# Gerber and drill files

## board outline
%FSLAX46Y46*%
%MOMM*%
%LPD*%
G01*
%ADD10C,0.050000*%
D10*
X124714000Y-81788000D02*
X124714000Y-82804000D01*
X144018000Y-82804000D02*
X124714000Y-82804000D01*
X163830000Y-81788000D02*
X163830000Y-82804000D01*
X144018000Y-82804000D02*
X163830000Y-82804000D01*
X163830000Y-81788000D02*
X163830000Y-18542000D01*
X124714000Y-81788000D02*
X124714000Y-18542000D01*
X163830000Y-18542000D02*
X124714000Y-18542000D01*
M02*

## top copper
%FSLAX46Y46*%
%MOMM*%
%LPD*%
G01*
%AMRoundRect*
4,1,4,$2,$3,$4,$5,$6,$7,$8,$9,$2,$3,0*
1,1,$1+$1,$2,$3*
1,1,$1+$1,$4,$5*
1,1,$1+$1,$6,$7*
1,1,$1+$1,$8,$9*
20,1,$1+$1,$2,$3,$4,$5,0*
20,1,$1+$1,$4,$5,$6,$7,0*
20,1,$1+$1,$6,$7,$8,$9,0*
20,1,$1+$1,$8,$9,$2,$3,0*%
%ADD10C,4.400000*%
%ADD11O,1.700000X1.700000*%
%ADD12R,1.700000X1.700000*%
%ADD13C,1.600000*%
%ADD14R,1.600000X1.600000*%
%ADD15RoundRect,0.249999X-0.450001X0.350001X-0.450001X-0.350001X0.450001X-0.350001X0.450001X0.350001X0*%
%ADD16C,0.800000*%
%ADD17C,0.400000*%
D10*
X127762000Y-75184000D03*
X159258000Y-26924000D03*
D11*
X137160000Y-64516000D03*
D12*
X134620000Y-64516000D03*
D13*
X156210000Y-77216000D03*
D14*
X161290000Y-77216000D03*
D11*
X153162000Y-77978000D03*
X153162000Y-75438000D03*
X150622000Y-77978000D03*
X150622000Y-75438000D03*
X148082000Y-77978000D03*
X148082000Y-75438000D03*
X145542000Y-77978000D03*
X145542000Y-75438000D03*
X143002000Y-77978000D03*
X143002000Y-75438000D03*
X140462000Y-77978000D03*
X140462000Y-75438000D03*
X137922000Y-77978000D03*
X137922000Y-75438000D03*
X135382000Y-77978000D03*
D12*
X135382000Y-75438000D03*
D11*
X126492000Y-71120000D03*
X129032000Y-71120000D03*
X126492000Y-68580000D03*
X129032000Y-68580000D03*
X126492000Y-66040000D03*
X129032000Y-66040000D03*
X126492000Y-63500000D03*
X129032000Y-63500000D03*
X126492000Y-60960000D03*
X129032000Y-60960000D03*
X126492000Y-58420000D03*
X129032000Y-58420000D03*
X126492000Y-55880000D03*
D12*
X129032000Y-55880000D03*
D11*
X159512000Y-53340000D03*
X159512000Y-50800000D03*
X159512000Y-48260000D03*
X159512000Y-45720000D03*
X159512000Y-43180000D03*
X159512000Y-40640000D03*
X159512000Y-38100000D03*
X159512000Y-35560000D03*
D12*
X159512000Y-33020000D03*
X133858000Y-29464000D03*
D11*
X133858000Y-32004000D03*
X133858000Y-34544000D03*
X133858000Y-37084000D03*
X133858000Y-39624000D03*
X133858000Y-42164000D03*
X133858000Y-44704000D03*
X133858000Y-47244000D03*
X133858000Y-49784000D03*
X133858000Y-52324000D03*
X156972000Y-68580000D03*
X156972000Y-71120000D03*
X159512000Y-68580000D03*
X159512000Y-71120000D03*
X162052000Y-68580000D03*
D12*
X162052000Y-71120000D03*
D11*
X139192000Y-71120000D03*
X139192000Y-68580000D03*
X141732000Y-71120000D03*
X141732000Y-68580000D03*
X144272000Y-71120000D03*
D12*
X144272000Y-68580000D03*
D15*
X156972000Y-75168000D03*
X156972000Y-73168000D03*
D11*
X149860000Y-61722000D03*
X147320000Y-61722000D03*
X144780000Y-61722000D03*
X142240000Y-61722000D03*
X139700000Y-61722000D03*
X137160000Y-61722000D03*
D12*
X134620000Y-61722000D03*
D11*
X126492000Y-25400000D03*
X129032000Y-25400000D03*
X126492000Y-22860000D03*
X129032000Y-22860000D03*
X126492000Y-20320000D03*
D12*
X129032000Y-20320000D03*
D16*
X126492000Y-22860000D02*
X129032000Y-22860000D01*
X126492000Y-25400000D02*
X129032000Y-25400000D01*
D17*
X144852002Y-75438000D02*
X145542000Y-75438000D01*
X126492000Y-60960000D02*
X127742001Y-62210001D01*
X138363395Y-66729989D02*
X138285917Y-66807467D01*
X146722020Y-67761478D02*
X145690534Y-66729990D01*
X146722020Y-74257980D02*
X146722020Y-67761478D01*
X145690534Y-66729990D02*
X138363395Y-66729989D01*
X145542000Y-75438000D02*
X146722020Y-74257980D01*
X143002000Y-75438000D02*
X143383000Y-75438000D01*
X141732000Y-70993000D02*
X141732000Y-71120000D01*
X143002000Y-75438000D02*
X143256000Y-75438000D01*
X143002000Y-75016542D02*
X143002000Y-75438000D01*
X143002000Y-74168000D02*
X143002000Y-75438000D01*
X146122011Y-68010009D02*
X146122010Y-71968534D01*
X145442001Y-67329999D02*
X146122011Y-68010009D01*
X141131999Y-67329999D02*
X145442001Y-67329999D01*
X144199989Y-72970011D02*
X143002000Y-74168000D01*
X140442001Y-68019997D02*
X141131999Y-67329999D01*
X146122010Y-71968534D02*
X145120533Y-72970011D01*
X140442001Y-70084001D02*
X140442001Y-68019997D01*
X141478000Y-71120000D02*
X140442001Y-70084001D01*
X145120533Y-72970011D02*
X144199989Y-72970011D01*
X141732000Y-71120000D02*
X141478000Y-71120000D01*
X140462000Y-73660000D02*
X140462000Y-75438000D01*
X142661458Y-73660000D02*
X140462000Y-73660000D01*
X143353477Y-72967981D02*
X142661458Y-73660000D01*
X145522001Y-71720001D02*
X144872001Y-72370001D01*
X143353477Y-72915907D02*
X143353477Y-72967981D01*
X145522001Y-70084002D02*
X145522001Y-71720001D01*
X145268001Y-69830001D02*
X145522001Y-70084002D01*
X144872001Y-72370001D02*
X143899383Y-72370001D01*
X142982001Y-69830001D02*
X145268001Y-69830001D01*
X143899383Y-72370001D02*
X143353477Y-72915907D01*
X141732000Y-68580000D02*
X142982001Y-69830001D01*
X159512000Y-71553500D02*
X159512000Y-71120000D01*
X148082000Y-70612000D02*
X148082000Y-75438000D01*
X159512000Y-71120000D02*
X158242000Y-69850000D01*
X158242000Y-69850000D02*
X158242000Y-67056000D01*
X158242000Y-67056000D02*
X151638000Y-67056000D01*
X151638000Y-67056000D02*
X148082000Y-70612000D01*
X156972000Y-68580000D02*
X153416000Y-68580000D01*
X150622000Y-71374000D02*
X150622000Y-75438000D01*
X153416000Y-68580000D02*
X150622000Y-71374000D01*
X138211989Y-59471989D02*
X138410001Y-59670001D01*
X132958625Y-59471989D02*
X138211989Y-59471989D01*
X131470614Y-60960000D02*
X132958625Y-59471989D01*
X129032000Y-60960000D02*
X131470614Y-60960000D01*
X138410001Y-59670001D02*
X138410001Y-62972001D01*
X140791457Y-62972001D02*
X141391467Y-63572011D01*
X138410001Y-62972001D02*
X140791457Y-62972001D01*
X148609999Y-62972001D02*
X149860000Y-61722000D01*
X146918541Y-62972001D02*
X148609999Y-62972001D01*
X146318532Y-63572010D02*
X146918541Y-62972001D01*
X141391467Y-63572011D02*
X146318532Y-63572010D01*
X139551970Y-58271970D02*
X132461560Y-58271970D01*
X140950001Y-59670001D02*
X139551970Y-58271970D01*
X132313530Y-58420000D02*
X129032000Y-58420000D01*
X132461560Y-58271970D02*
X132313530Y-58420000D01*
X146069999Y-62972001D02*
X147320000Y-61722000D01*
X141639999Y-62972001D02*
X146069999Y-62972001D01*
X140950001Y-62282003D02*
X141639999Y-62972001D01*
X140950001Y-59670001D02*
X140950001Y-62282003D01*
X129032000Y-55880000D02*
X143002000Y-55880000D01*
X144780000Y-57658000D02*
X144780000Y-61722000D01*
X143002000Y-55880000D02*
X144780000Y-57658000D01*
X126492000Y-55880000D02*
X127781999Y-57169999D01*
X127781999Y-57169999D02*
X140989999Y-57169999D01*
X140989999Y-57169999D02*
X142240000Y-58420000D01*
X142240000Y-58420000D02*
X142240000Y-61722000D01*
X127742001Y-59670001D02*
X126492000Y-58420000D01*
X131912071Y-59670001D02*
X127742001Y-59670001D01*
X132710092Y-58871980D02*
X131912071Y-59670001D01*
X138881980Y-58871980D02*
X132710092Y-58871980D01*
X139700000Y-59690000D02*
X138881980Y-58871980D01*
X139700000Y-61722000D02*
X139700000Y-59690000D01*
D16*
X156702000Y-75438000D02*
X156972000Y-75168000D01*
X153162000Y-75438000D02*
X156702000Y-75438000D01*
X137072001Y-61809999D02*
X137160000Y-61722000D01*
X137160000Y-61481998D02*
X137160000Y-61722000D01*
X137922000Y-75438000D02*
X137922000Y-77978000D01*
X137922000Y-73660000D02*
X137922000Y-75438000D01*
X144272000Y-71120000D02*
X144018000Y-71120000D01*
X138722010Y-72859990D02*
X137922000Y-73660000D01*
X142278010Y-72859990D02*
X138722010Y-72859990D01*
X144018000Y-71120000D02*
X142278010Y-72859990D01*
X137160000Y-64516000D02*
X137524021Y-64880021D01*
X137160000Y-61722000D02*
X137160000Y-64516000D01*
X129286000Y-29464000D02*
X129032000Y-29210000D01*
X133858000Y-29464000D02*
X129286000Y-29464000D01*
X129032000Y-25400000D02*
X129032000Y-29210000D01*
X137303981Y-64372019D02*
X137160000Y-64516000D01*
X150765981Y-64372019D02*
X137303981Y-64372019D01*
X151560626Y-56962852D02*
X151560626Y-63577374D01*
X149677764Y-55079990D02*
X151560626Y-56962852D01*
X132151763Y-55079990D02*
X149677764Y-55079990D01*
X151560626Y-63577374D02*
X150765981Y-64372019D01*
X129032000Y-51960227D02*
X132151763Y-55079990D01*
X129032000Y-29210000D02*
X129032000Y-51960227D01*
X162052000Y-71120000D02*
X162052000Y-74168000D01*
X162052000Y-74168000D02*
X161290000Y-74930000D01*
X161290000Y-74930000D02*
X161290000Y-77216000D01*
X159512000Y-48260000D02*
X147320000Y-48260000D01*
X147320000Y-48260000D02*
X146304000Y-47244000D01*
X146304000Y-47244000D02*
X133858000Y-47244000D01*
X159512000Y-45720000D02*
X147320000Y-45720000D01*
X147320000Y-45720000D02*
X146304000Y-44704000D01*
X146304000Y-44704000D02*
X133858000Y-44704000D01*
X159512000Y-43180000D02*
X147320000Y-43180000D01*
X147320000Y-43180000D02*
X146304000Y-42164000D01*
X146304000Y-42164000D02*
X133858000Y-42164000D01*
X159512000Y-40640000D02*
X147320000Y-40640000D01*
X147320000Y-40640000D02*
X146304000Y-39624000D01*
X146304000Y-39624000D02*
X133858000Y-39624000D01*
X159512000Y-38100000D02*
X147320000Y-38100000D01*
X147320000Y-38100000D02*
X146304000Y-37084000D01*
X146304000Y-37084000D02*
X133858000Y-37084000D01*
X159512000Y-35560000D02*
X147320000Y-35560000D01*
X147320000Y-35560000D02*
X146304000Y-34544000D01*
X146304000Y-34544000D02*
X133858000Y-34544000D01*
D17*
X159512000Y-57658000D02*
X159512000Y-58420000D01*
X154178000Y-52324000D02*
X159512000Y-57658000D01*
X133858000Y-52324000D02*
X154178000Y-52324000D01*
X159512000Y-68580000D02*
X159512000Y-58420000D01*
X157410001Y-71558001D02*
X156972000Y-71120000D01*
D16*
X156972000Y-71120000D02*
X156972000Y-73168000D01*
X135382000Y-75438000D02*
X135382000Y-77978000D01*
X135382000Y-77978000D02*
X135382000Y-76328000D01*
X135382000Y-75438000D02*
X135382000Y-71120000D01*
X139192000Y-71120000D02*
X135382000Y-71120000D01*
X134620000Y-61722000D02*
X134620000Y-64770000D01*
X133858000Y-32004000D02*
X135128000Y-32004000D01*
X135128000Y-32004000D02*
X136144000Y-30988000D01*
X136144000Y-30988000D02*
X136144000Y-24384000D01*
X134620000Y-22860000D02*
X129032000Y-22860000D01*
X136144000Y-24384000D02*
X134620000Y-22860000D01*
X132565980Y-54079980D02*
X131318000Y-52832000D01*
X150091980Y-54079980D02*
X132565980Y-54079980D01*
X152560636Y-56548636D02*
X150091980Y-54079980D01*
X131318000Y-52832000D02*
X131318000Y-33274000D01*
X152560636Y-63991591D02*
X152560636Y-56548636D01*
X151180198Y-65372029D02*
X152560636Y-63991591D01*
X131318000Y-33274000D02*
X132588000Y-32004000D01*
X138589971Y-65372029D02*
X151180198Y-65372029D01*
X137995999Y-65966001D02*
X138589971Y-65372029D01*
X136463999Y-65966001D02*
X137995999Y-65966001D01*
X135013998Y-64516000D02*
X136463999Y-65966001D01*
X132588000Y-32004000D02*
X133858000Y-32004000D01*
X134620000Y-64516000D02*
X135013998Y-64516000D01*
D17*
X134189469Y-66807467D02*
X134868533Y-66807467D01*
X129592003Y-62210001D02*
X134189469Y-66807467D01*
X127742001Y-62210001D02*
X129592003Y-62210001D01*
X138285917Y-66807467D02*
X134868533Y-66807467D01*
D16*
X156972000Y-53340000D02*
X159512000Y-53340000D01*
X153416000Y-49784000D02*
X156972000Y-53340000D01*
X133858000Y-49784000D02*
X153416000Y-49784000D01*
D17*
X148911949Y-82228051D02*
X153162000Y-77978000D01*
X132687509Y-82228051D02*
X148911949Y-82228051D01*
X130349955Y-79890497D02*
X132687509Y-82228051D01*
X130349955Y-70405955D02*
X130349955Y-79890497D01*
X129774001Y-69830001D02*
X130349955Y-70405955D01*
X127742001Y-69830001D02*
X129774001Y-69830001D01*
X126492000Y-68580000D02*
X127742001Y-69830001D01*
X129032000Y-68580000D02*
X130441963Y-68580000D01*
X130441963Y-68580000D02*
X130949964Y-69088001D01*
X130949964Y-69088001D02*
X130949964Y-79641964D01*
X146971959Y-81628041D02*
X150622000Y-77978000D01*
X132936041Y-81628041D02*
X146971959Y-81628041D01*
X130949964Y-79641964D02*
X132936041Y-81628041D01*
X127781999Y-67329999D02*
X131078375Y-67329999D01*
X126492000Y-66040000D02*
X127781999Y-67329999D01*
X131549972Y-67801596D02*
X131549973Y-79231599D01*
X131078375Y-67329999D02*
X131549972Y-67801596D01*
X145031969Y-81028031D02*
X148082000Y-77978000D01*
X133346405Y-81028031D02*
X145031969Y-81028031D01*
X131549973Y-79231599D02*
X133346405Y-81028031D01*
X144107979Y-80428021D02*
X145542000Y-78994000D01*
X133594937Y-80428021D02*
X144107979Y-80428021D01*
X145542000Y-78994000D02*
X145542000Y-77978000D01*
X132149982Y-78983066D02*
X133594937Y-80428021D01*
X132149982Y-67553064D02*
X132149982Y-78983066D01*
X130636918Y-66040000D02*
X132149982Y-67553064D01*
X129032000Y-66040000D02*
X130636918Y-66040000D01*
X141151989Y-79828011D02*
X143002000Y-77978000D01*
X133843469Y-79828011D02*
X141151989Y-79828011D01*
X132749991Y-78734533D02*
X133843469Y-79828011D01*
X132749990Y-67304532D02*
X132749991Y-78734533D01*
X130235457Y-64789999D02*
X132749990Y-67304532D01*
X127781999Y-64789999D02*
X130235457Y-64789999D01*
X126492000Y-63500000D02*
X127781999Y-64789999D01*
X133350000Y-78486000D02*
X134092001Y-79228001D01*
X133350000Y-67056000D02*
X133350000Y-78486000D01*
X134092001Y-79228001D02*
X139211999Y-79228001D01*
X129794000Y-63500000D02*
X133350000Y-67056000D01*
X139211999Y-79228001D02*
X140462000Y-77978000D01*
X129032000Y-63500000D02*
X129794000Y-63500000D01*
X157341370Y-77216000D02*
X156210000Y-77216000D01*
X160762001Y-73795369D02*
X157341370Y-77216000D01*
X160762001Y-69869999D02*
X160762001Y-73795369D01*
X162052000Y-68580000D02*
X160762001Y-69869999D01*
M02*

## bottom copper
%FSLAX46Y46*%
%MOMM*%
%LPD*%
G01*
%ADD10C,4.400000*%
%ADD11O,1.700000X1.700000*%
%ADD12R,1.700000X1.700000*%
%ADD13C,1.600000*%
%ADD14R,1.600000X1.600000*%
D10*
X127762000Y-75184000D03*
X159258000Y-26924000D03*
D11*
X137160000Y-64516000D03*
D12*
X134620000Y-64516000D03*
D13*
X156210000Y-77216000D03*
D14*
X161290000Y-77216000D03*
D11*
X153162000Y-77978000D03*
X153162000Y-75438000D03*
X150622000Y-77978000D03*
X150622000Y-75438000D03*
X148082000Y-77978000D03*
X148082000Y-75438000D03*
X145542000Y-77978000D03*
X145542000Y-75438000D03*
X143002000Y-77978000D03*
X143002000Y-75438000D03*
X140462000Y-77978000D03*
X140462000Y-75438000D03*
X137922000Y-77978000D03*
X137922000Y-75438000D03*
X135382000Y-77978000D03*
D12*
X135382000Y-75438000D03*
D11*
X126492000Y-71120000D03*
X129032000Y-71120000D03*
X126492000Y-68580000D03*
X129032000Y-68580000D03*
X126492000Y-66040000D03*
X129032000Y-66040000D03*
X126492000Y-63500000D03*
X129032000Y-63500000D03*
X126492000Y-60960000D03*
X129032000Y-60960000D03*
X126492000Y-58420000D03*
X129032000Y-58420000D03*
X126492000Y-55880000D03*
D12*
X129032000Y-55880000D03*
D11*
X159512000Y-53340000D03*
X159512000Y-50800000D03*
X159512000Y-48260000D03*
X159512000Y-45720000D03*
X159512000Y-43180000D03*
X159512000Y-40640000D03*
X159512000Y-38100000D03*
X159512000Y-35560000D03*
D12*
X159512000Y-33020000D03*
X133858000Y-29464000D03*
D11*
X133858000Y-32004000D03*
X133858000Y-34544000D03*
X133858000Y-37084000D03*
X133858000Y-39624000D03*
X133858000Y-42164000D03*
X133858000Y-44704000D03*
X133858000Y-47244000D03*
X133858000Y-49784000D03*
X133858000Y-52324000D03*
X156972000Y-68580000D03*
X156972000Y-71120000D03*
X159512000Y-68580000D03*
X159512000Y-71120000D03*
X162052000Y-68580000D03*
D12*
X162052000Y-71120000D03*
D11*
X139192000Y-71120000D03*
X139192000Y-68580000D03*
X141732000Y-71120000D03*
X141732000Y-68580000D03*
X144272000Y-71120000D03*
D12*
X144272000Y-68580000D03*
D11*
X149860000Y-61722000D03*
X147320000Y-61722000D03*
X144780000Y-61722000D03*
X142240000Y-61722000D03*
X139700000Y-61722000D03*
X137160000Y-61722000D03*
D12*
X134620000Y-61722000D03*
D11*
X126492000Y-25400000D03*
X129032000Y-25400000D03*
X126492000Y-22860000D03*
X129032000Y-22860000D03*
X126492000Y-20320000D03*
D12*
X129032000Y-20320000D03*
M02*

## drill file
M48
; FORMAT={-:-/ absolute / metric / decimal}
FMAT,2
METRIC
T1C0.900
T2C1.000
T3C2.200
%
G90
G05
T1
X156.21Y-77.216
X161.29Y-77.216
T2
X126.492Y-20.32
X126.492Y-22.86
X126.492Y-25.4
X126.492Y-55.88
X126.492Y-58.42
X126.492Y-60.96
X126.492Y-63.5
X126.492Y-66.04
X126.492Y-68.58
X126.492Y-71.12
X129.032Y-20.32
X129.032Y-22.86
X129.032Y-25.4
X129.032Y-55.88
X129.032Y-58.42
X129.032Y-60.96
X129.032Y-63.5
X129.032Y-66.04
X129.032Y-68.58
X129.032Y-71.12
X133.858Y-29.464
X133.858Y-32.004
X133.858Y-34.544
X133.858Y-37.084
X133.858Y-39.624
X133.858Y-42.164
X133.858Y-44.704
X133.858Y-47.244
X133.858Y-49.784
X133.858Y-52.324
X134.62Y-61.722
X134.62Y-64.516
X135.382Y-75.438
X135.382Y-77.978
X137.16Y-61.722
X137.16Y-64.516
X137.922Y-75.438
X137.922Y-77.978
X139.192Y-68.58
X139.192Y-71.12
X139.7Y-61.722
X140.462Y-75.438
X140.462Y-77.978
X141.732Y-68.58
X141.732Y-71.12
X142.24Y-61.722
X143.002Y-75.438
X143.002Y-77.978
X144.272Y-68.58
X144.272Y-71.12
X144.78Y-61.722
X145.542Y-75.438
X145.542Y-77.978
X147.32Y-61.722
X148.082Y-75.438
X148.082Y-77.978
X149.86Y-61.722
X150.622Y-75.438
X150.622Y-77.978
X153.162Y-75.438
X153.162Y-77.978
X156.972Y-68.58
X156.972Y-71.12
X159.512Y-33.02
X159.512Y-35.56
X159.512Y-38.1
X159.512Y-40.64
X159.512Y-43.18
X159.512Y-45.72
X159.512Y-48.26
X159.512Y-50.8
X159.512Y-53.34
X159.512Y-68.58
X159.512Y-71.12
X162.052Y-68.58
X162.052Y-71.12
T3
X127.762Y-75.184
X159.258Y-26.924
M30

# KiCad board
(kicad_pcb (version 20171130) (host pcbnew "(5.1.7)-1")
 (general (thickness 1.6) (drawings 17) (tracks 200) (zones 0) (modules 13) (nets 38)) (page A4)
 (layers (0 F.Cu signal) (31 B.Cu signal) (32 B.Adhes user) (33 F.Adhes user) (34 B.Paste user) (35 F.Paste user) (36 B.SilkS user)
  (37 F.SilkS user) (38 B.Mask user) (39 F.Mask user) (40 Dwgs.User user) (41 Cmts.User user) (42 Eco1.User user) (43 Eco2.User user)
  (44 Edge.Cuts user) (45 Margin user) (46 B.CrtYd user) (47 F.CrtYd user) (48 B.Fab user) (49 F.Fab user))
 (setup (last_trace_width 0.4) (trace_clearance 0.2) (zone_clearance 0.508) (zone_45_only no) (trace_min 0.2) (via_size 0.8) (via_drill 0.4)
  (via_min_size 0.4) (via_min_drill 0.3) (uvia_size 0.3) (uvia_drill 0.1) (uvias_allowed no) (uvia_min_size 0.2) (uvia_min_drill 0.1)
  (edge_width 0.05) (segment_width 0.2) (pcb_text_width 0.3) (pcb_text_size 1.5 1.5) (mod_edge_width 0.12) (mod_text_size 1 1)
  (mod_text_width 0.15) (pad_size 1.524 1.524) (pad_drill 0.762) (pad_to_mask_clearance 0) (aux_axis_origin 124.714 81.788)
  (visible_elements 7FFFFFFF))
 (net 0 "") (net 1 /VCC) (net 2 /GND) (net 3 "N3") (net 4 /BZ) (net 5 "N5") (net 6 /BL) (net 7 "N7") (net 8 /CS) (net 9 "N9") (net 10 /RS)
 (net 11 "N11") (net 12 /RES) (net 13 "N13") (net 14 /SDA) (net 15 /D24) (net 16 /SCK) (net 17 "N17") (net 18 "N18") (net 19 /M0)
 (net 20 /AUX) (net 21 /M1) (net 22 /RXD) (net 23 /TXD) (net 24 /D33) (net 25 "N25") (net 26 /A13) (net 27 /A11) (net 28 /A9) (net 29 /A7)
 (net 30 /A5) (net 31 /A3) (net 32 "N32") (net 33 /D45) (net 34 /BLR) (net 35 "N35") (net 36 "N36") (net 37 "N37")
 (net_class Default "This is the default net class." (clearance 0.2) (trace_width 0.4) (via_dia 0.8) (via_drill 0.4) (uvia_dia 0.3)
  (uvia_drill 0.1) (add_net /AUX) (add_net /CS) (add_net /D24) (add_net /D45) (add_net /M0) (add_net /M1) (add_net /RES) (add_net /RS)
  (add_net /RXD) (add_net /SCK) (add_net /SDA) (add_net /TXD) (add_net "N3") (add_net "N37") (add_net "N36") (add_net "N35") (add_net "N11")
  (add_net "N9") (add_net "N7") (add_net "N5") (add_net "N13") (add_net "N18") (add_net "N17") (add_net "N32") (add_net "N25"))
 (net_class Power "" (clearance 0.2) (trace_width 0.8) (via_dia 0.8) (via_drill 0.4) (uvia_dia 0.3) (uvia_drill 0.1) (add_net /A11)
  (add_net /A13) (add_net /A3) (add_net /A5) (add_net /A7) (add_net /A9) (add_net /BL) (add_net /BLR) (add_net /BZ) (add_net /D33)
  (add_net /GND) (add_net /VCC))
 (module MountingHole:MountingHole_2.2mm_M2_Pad (layer F.Cu) (at 127.762 75.184)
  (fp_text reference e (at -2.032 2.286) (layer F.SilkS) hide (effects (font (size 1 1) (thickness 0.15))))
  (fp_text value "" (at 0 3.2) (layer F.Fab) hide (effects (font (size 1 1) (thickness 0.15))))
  (pad 1 thru_hole circle (at 0 0) (size 4.4 4.4) (drill 2.2) (layers *.Cu *.Mask)))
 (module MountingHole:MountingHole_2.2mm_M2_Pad (layer F.Cu) (at 159.258 26.924)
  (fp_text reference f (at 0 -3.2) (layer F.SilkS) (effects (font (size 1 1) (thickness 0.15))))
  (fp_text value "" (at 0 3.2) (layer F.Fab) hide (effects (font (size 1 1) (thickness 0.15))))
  (pad 1 thru_hole circle (at 0 0) (size 4.4 4.4) (drill 2.2) (layers *.Cu *.Mask)))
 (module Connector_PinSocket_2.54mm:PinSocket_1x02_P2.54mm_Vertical (layer F.Cu) (at 134.62 64.516 90)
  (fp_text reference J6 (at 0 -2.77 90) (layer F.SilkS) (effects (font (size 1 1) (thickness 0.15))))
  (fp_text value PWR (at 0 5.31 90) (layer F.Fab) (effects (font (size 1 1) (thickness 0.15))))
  (pad 2 thru_hole oval (at 0 2.54 90) (size 1.7 1.7) (drill 1) (layers *.Cu *.Mask) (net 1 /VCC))
  (pad 1 thru_hole rect (at 0 0 90) (size 1.7 1.7) (drill 1) (layers *.Cu *.Mask) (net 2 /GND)))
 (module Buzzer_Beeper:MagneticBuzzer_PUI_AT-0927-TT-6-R (layer F.Cu) (at 160.782 77.216 180)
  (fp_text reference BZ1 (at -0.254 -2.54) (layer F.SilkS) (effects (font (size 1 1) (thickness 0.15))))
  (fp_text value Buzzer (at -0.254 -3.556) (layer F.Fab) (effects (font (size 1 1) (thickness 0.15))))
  (pad 2 thru_hole circle (at 4.572 0 180) (size 1.6 1.6) (drill 0.9) (layers *.Cu *.Mask) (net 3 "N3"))
  (pad 1 thru_hole rect (at -0.508 0 180) (size 1.6 1.6) (drill 0.9) (layers *.Cu *.Mask) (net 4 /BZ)))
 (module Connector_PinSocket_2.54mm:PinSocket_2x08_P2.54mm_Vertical (layer F.Cu) (at 135.382 75.438 90)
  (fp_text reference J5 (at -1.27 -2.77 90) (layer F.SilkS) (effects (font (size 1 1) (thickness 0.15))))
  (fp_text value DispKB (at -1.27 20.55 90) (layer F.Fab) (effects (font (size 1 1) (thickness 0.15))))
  (pad 16 thru_hole oval (at -2.54 17.78 90) (size 1.7 1.7) (drill 1) (layers *.Cu *.Mask) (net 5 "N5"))
  (pad 15 thru_hole oval (at 0 17.78 90) (size 1.7 1.7) (drill 1) (layers *.Cu *.Mask) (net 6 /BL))
  (pad 14 thru_hole oval (at -2.54 15.24 90) (size 1.7 1.7) (drill 1) (layers *.Cu *.Mask) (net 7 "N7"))
  (pad 13 thru_hole oval (at 0 15.24 90) (size 1.7 1.7) (drill 1) (layers *.Cu *.Mask) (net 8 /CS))
  (pad 12 thru_hole oval (at -2.54 12.7 90) (size 1.7 1.7) (drill 1) (layers *.Cu *.Mask) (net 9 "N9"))
  (pad 11 thru_hole oval (at 0 12.7 90) (size 1.7 1.7) (drill 1) (layers *.Cu *.Mask) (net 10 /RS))
  (pad 10 thru_hole oval (at -2.54 10.16 90) (size 1.7 1.7) (drill 1) (layers *.Cu *.Mask) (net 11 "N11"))
  (pad 9 thru_hole oval (at 0 10.16 90) (size 1.7 1.7) (drill 1) (layers *.Cu *.Mask) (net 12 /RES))
  (pad 8 thru_hole oval (at -2.54 7.62 90) (size 1.7 1.7) (drill 1) (layers *.Cu *.Mask) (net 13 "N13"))
  (pad 7 thru_hole oval (at 0 7.62 90) (size 1.7 1.7) (drill 1) (layers *.Cu *.Mask) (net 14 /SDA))
  (pad 6 thru_hole oval (at -2.54 5.08 90) (size 1.7 1.7) (drill 1) (layers *.Cu *.Mask) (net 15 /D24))
  (pad 5 thru_hole oval (at 0 5.08 90) (size 1.7 1.7) (drill 1) (layers *.Cu *.Mask) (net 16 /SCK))
  (pad 4 thru_hole oval (at -2.54 2.54 90) (size 1.7 1.7) (drill 1) (layers *.Cu *.Mask) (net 1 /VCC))
  (pad 3 thru_hole oval (at 0 2.54 90) (size 1.7 1.7) (drill 1) (layers *.Cu *.Mask) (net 1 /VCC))
  (pad 2 thru_hole oval (at -2.54 0 90) (size 1.7 1.7) (drill 1) (layers *.Cu *.Mask) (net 2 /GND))
  (pad 1 thru_hole rect (at 0 0 90) (size 1.7 1.7) (drill 1) (layers *.Cu *.Mask) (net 2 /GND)))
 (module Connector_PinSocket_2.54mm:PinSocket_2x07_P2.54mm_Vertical (layer F.Cu) (at 129.032 55.88)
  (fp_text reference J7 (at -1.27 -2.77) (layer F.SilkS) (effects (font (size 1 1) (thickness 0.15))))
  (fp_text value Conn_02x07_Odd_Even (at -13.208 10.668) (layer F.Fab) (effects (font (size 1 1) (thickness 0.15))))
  (pad 14 thru_hole oval (at -2.54 15.24) (size 1.7 1.7) (drill 1) (layers *.Cu *.Mask) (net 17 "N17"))
  (pad 13 thru_hole oval (at 0 15.24) (size 1.7 1.7) (drill 1) (layers *.Cu *.Mask) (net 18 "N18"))
  (pad 12 thru_hole oval (at -2.54 12.7) (size 1.7 1.7) (drill 1) (layers *.Cu *.Mask) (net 5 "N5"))
  (pad 11 thru_hole oval (at 0 12.7) (size 1.7 1.7) (drill 1) (layers *.Cu *.Mask) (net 7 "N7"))
  (pad 10 thru_hole oval (at -2.54 10.16) (size 1.7 1.7) (drill 1) (layers *.Cu *.Mask) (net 9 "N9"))
  (pad 9 thru_hole oval (at 0 10.16) (size 1.7 1.7) (drill 1) (layers *.Cu *.Mask) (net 11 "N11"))
  (pad 8 thru_hole oval (at -2.54 7.62) (size 1.7 1.7) (drill 1) (layers *.Cu *.Mask) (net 13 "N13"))
  (pad 7 thru_hole oval (at 0 7.62) (size 1.7 1.7) (drill 1) (layers *.Cu *.Mask) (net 15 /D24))
  (pad 6 thru_hole oval (at -2.54 5.08) (size 1.7 1.7) (drill 1) (layers *.Cu *.Mask) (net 12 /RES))
  (pad 5 thru_hole oval (at 0 5.08) (size 1.7 1.7) (drill 1) (layers *.Cu *.Mask) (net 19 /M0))
  (pad 4 thru_hole oval (at -2.54 2.54) (size 1.7 1.7) (drill 1) (layers *.Cu *.Mask) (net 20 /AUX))
  (pad 3 thru_hole oval (at 0 2.54) (size 1.7 1.7) (drill 1) (layers *.Cu *.Mask) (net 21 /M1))
  (pad 2 thru_hole oval (at -2.54 0) (size 1.7 1.7) (drill 1) (layers *.Cu *.Mask) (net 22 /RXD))
  (pad 1 thru_hole rect (at 0 0) (size 1.7 1.7) (drill 1) (layers *.Cu *.Mask) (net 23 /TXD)))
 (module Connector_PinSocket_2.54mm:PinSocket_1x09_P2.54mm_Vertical (layer F.Cu) (at 159.512 33.02)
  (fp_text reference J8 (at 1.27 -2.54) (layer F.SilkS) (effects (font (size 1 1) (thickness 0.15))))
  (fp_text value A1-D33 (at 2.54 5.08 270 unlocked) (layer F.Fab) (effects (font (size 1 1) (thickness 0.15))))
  (pad 9 thru_hole oval (at 0 20.32) (size 1.7 1.7) (drill 1) (layers *.Cu *.Mask) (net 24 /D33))
  (pad 8 thru_hole oval (at 0 17.78) (size 1.7 1.7) (drill 1) (layers *.Cu *.Mask) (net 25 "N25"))
  (pad 7 thru_hole oval (at 0 15.24) (size 1.7 1.7) (drill 1) (layers *.Cu *.Mask) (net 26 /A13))
  (pad 6 thru_hole oval (at 0 12.7) (size 1.7 1.7) (drill 1) (layers *.Cu *.Mask) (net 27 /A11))
  (pad 5 thru_hole oval (at 0 10.16) (size 1.7 1.7) (drill 1) (layers *.Cu *.Mask) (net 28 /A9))
  (pad 4 thru_hole oval (at 0 7.62) (size 1.7 1.7) (drill 1) (layers *.Cu *.Mask) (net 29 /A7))
  (pad 3 thru_hole oval (at 0 5.08) (size 1.7 1.7) (drill 1) (layers *.Cu *.Mask) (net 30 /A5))
  (pad 2 thru_hole oval (at 0 2.54) (size 1.7 1.7) (drill 1) (layers *.Cu *.Mask) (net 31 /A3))
  (pad 1 thru_hole rect (at 0 0) (size 1.7 1.7) (drill 1) (layers *.Cu *.Mask) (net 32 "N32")))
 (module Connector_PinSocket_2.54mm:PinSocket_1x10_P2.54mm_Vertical (layer F.Cu) (at 133.858 29.464)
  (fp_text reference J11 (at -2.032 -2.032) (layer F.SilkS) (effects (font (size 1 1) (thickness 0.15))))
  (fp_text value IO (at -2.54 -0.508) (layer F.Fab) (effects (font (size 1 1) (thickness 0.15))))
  (pad 1 thru_hole rect (at 0 0) (size 1.7 1.7) (drill 1) (layers *.Cu *.Mask) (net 1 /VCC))
  (pad 2 thru_hole oval (at 0 2.54) (size 1.7 1.7) (drill 1) (layers *.Cu *.Mask) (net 2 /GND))
  (pad 3 thru_hole oval (at 0 5.08) (size 1.7 1.7) (drill 1) (layers *.Cu *.Mask) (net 31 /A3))
  (pad 4 thru_hole oval (at 0 7.62) (size 1.7 1.7) (drill 1) (layers *.Cu *.Mask) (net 30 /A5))
  (pad 5 thru_hole oval (at 0 10.16) (size 1.7 1.7) (drill 1) (layers *.Cu *.Mask) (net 29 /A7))
  (pad 6 thru_hole oval (at 0 12.7) (size 1.7 1.7) (drill 1) (layers *.Cu *.Mask) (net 28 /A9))
  (pad 7 thru_hole oval (at 0 15.24) (size 1.7 1.7) (drill 1) (layers *.Cu *.Mask) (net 27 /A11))
  (pad 8 thru_hole oval (at 0 17.78) (size 1.7 1.7) (drill 1) (layers *.Cu *.Mask) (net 26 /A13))
  (pad 9 thru_hole oval (at 0 20.32) (size 1.7 1.7) (drill 1) (layers *.Cu *.Mask) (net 24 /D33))
  (pad 10 thru_hole oval (at 0 22.86) (size 1.7 1.7) (drill 1) (layers *.Cu *.Mask) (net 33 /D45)))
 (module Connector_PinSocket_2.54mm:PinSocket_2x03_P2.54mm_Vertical (layer F.Cu) (at 162.052 71.12 270)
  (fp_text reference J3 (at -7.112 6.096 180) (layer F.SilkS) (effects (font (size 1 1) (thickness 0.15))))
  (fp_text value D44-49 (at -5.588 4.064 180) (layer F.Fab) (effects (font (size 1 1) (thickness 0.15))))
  (pad 6 thru_hole oval (at -2.54 5.08 270) (size 1.7 1.7) (drill 1) (layers *.Cu *.Mask) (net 8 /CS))
  (pad 5 thru_hole oval (at 0 5.08 270) (size 1.7 1.7) (drill 1) (layers *.Cu *.Mask) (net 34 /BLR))
  (pad 4 thru_hole oval (at -2.54 2.54 270) (size 1.7 1.7) (drill 1) (layers *.Cu *.Mask) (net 33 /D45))
  (pad 3 thru_hole oval (at 0 2.54 270) (size 1.7 1.7) (drill 1) (layers *.Cu *.Mask) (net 10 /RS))
  (pad 2 thru_hole oval (at -2.54 0 270) (size 1.7 1.7) (drill 1) (layers *.Cu *.Mask) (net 3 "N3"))
  (pad 1 thru_hole rect (at 0 0 270) (size 1.7 1.7) (drill 1) (layers *.Cu *.Mask) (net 4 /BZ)))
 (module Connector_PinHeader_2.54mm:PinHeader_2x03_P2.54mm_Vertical (layer F.Cu) (at 144.272 68.58 270)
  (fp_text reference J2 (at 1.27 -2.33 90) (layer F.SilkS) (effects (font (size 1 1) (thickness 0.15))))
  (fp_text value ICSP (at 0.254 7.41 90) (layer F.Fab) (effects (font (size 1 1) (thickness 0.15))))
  (pad 6 thru_hole oval (at 2.54 5.08 270) (size 1.7 1.7) (drill 1) (layers *.Cu *.Mask) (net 2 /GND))
  (pad 5 thru_hole oval (at 0 5.08 270) (size 1.7 1.7) (drill 1) (layers *.Cu *.Mask) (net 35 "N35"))
  (pad 4 thru_hole oval (at 2.54 2.54 270) (size 1.7 1.7) (drill 1) (layers *.Cu *.Mask) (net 14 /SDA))
  (pad 3 thru_hole oval (at 0 2.54 270) (size 1.7 1.7) (drill 1) (layers *.Cu *.Mask) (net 16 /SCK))
  (pad 2 thru_hole oval (at 2.54 0 270) (size 1.7 1.7) (drill 1) (layers *.Cu *.Mask) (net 1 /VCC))
  (pad 1 thru_hole rect (at 0 0 270) (size 1.7 1.7) (drill 1) (layers *.Cu *.Mask) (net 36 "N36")))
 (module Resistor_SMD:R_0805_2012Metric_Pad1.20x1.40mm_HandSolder (layer F.Cu) (at 156.972 74.168 270)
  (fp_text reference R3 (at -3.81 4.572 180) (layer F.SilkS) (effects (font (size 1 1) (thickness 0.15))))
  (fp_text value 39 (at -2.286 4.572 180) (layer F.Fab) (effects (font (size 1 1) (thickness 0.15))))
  (pad 2 smd roundrect (at 1 0 270) (size 1.2 1.4) (layers F.Cu F.Paste F.Mask) (roundrect_rratio 0.2083325) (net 6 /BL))
  (pad 1 smd roundrect (at -1 0 270) (size 1.2 1.4) (layers F.Cu F.Paste F.Mask) (roundrect_rratio 0.2083325) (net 34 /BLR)))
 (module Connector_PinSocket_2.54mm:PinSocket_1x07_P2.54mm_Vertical (layer F.Cu) (at 134.62 61.722 90)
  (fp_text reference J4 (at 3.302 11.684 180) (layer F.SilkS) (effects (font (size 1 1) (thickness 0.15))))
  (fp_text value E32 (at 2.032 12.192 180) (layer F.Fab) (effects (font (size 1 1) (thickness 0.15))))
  (pad 7 thru_hole oval (at 0 15.24 90) (size 1.7 1.7) (drill 1) (layers *.Cu *.Mask) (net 19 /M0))
  (pad 6 thru_hole oval (at 0 12.7 90) (size 1.7 1.7) (drill 1) (layers *.Cu *.Mask) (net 21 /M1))
  (pad 5 thru_hole oval (at 0 10.16 90) (size 1.7 1.7) (drill 1) (layers *.Cu *.Mask) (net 23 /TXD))
  (pad 4 thru_hole oval (at 0 7.62 90) (size 1.7 1.7) (drill 1) (layers *.Cu *.Mask) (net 22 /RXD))
  (pad 3 thru_hole oval (at 0 5.08 90) (size 1.7 1.7) (drill 1) (layers *.Cu *.Mask) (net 20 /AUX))
  (pad 2 thru_hole oval (at 0 2.54 90) (size 1.7 1.7) (drill 1) (layers *.Cu *.Mask) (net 1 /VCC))
  (pad 1 thru_hole rect (at 0 0 90) (size 1.7 1.7) (drill 1) (layers *.Cu *.Mask) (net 2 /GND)))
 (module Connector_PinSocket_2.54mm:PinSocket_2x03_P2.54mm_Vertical (layer F.Cu) (at 129.032 20.32)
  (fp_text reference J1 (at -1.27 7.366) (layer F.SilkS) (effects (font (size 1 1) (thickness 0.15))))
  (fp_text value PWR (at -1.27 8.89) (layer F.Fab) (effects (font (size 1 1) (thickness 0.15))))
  (pad 6 thru_hole oval (at -2.54 5.08) (size 1.7 1.7) (drill 1) (layers *.Cu *.Mask) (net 1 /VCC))
  (pad 5 thru_hole oval (at 0 5.08) (size 1.7 1.7) (drill 1) (layers *.Cu *.Mask) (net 1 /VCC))
  (pad 4 thru_hole oval (at -2.54 2.54) (size 1.7 1.7) (drill 1) (layers *.Cu *.Mask) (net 2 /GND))
  (pad 3 thru_hole oval (at 0 2.54) (size 1.7 1.7) (drill 1) (layers *.Cu *.Mask) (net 2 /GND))
  (pad 2 thru_hole oval (at -2.54 0) (size 1.7 1.7) (drill 1) (layers *.Cu *.Mask) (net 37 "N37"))
  (pad 1 thru_hole rect (at 0 0) (size 1.7 1.7) (drill 1) (layers *.Cu *.Mask) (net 37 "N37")))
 (gr_line (start 124.714 81.788) (end 124.714 82.804) (layer Edge.Cuts) (width 0.05))
 (gr_line (start 144.018 82.804) (end 124.714 82.804) (layer Edge.Cuts) (width 0.05))
 (gr_line (start 163.83 81.788) (end 163.83 82.804) (layer Edge.Cuts) (width 0.05))
 (gr_line (start 144.018 82.804) (end 163.83 82.804) (layer Edge.Cuts) (width 0.05))
 (gr_line (start 163.83 81.788) (end 163.83 18.542) (layer Edge.Cuts) (width 0.05))
 (gr_line (start 124.714 81.788) (end 124.714 18.542) (layer Edge.Cuts) (width 0.05))
 (gr_line (start 163.83 18.542) (end 124.714 18.542) (layer Edge.Cuts) (width 0.05))
 (segment (start 126.492 22.86) (end 129.032 22.86) (width 0.8) (layer F.Cu) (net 2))
 (segment (start 126.492 25.4) (end 129.032 25.4) (width 0.8) (layer F.Cu) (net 1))
 (segment (start 144.852002 75.438) (end 145.542 75.438) (width 0.4) (layer F.Cu) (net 12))
 (segment (start 126.492 60.96) (end 127.742001 62.210001) (width 0.4) (layer F.Cu) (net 12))
 (segment (start 138.363395 66.729989) (end 138.285917 66.807467) (width 0.4) (layer F.Cu) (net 12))
 (segment (start 146.72202 67.761478) (end 145.690534 66.72999) (width 0.4) (layer F.Cu) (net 12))
 (segment (start 146.72202 74.25798) (end 146.72202 67.761478) (width 0.4) (layer F.Cu) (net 12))
 (segment (start 145.690534 66.72999) (end 138.363395 66.729989) (width 0.4) (layer F.Cu) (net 12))
 (segment (start 145.542 75.438) (end 146.72202 74.25798) (width 0.4) (layer F.Cu) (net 12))
 (segment (start 143.002 75.438) (end 143.383 75.438) (width 0.4) (layer F.Cu) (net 14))
 (segment (start 141.732 70.993) (end 141.732 71.12) (width 0.4) (layer F.Cu) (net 14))
 (segment (start 143.002 75.438) (end 143.256 75.438) (width 0.4) (layer F.Cu) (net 14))
 (segment (start 143.002 75.016542) (end 143.002 75.438) (width 0.4) (layer F.Cu) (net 14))
 (segment (start 143.002 74.168) (end 143.002 75.438) (width 0.4) (layer F.Cu) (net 14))
 (segment (start 146.122011 68.010009) (end 146.12201 71.968534) (width 0.4) (layer F.Cu) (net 14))
 (segment (start 145.442001 67.329999) (end 146.122011 68.010009) (width 0.4) (layer F.Cu) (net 14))
 (segment (start 141.131999 67.329999) (end 145.442001 67.329999) (width 0.4) (layer F.Cu) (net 14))
 (segment (start 144.199989 72.970011) (end 143.002 74.168) (width 0.4) (layer F.Cu) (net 14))
 (segment (start 140.442001 68.019997) (end 141.131999 67.329999) (width 0.4) (layer F.Cu) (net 14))
 (segment (start 146.12201 71.968534) (end 145.120533 72.970011) (width 0.4) (layer F.Cu) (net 14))
 (segment (start 140.442001 70.084001) (end 140.442001 68.019997) (width 0.4) (layer F.Cu) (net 14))
 (segment (start 141.478 71.12) (end 140.442001 70.084001) (width 0.4) (layer F.Cu) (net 14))
 (segment (start 145.120533 72.970011) (end 144.199989 72.970011) (width 0.4) (layer F.Cu) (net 14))
 (segment (start 141.732 71.12) (end 141.478 71.12) (width 0.4) (layer F.Cu) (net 14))
 (segment (start 140.462 73.66) (end 140.462 75.438) (width 0.4) (layer F.Cu) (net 16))
 (segment (start 142.661458 73.66) (end 140.462 73.66) (width 0.4) (layer F.Cu) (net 16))
 (segment (start 143.353477 72.967981) (end 142.661458 73.66) (width 0.4) (layer F.Cu) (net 16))
 (segment (start 145.522001 71.720001) (end 144.872001 72.370001) (width 0.4) (layer F.Cu) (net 16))
 (segment (start 143.353477 72.915907) (end 143.353477 72.967981) (width 0.4) (layer F.Cu) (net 16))
 (segment (start 145.522001 70.084002) (end 145.522001 71.720001) (width 0.4) (layer F.Cu) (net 16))
 (segment (start 145.268001 69.830001) (end 145.522001 70.084002) (width 0.4) (layer F.Cu) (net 16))
 (segment (start 144.872001 72.370001) (end 143.899383 72.370001) (width 0.4) (layer F.Cu) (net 16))
 (segment (start 142.982001 69.830001) (end 145.268001 69.830001) (width 0.4) (layer F.Cu) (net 16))
 (segment (start 143.899383 72.370001) (end 143.353477 72.915907) (width 0.4) (layer F.Cu) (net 16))
 (segment (start 141.732 68.58) (end 142.982001 69.830001) (width 0.4) (layer F.Cu) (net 16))
 (segment (start 159.512 71.5535) (end 159.512 71.12) (width 0.4) (layer F.Cu) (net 10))
 (segment (start 148.082 70.612) (end 148.082 75.438) (width 0.4) (layer F.Cu) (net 10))
 (segment (start 159.512 71.12) (end 158.242 69.85) (width 0.4) (layer F.Cu) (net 10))
 (segment (start 158.242 69.85) (end 158.242 67.056) (width 0.4) (layer F.Cu) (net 10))
 (segment (start 158.242 67.056) (end 151.638 67.056) (width 0.4) (layer F.Cu) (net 10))
 (segment (start 151.638 67.056) (end 148.082 70.612) (width 0.4) (layer F.Cu) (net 10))
 (segment (start 156.972 68.58) (end 153.416 68.58) (width 0.4) (layer F.Cu) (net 8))
 (segment (start 150.622 71.374) (end 150.622 75.438) (width 0.4) (layer F.Cu) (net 8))
 (segment (start 153.416 68.58) (end 150.622 71.374) (width 0.4) (layer F.Cu) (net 8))
 (segment (start 138.211989 59.471989) (end 138.410001 59.670001) (width 0.4) (layer F.Cu) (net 19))
 (segment (start 132.958625 59.471989) (end 138.211989 59.471989) (width 0.4) (layer F.Cu) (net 19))
 (segment (start 131.470614 60.96) (end 132.958625 59.471989) (width 0.4) (layer F.Cu) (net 19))
 (segment (start 129.032 60.96) (end 131.470614 60.96) (width 0.4) (layer F.Cu) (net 19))
 (segment (start 138.410001 59.670001) (end 138.410001 62.972001) (width 0.4) (layer F.Cu) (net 19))
 (segment (start 140.791457 62.972001) (end 141.391467 63.572011) (width 0.4) (layer F.Cu) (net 19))
 (segment (start 138.410001 62.972001) (end 140.791457 62.972001) (width 0.4) (layer F.Cu) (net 19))
 (segment (start 148.609999 62.972001) (end 149.86 61.722) (width 0.4) (layer F.Cu) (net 19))
 (segment (start 146.918541 62.972001) (end 148.609999 62.972001) (width 0.4) (layer F.Cu) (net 19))
 (segment (start 146.318532 63.57201) (end 146.918541 62.972001) (width 0.4) (layer F.Cu) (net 19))
 (segment (start 141.391467 63.572011) (end 146.318532 63.57201) (width 0.4) (layer F.Cu) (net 19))
 (segment (start 139.55197 58.27197) (end 132.46156 58.27197) (width 0.4) (layer F.Cu) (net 21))
 (segment (start 140.950001 59.670001) (end 139.55197 58.27197) (width 0.4) (layer F.Cu) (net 21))
 (segment (start 132.31353 58.42) (end 129.032 58.42) (width 0.4) (layer F.Cu) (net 21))
 (segment (start 132.46156 58.27197) (end 132.31353 58.42) (width 0.4) (layer F.Cu) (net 21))
 (segment (start 146.069999 62.972001) (end 147.32 61.722) (width 0.4) (layer F.Cu) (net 21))
 (segment (start 141.639999 62.972001) (end 146.069999 62.972001) (width 0.4) (layer F.Cu) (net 21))
 (segment (start 140.950001 62.282003) (end 141.639999 62.972001) (width 0.4) (layer F.Cu) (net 21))
 (segment (start 140.950001 59.670001) (end 140.950001 62.282003) (width 0.4) (layer F.Cu) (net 21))
 (segment (start 129.032 55.88) (end 143.002 55.88) (width 0.4) (layer F.Cu) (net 23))
 (segment (start 144.78 57.658) (end 144.78 61.722) (width 0.4) (layer F.Cu) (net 23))
 (segment (start 143.002 55.88) (end 144.78 57.658) (width 0.4) (layer F.Cu) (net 23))
 (segment (start 126.492 55.88) (end 127.781999 57.169999) (width 0.4) (layer F.Cu) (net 22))
 (segment (start 127.781999 57.169999) (end 140.989999 57.169999) (width 0.4) (layer F.Cu) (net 22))
 (segment (start 140.989999 57.169999) (end 142.24 58.42) (width 0.4) (layer F.Cu) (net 22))
 (segment (start 142.24 58.42) (end 142.24 61.722) (width 0.4) (layer F.Cu) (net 22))
 (segment (start 127.742001 59.670001) (end 126.492 58.42) (width 0.4) (layer F.Cu) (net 20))
 (segment (start 131.912071 59.670001) (end 127.742001 59.670001) (width 0.4) (layer F.Cu) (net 20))
 (segment (start 132.710092 58.87198) (end 131.912071 59.670001) (width 0.4) (layer F.Cu) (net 20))
 (segment (start 138.88198 58.87198) (end 132.710092 58.87198) (width 0.4) (layer F.Cu) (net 20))
 (segment (start 139.7 59.69) (end 138.88198 58.87198) (width 0.4) (layer F.Cu) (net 20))
 (segment (start 139.7 61.722) (end 139.7 59.69) (width 0.4) (layer F.Cu) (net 20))
 (segment (start 156.702 75.438) (end 156.972 75.168) (width 0.8) (layer F.Cu) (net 6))
 (segment (start 153.162 75.438) (end 156.702 75.438) (width 0.8) (layer F.Cu) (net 6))
 (segment (start 137.072001 61.809999) (end 137.16 61.722) (width 0.8) (layer F.Cu) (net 1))
 (segment (start 137.16 61.481998) (end 137.16 61.722) (width 0.8) (layer F.Cu) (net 1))
 (segment (start 137.922 75.438) (end 137.922 77.978) (width 0.8) (layer F.Cu) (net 1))
 (segment (start 137.922 73.66) (end 137.922 75.438) (width 0.8) (layer F.Cu) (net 1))
 (segment (start 144.272 71.12) (end 144.018 71.12) (width 0.8) (layer F.Cu) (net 1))
 (segment (start 138.72201 72.85999) (end 137.922 73.66) (width 0.8) (layer F.Cu) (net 1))
 (segment (start 142.27801 72.85999) (end 138.72201 72.85999) (width 0.8) (layer F.Cu) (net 1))
 (segment (start 144.018 71.12) (end 142.27801 72.85999) (width 0.8) (layer F.Cu) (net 1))
 (segment (start 137.16 64.516) (end 137.524021 64.880021) (width 0.8) (layer F.Cu) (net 1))
 (segment (start 137.16 61.722) (end 137.16 64.516) (width 0.8) (layer F.Cu) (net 1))
 (segment (start 129.286 29.464) (end 129.032 29.21) (width 0.8) (layer F.Cu) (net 1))
 (segment (start 133.858 29.464) (end 129.286 29.464) (width 0.8) (layer F.Cu) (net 1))
 (segment (start 129.032 25.4) (end 129.032 29.21) (width 0.8) (layer F.Cu) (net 1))
 (segment (start 137.303981 64.372019) (end 137.16 64.516) (width 0.8) (layer F.Cu) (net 1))
 (segment (start 150.765981 64.372019) (end 137.303981 64.372019) (width 0.8) (layer F.Cu) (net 1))
 (segment (start 151.560626 56.962852) (end 151.560626 63.577374) (width 0.8) (layer F.Cu) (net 1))
 (segment (start 149.677764 55.07999) (end 151.560626 56.962852) (width 0.8) (layer F.Cu) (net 1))
 (segment (start 132.151763 55.07999) (end 149.677764 55.07999) (width 0.8) (layer F.Cu) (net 1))
 (segment (start 151.560626 63.577374) (end 150.765981 64.372019) (width 0.8) (layer F.Cu) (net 1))
 (segment (start 129.032 51.960227) (end 132.151763 55.07999) (width 0.8) (layer F.Cu) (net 1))
 (segment (start 129.032 29.21) (end 129.032 51.960227) (width 0.8) (layer F.Cu) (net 1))
 (segment (start 162.052 71.12) (end 162.052 74.168) (width 0.8) (layer F.Cu) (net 4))
 (segment (start 162.052 74.168) (end 161.29 74.93) (width 0.8) (layer F.Cu) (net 4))
 (segment (start 161.29 74.93) (end 161.29 77.216) (width 0.8) (layer F.Cu) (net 4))
 (segment (start 159.512 48.26) (end 147.32 48.26) (width 0.8) (layer F.Cu) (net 26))
 (segment (start 147.32 48.26) (end 146.304 47.244) (width 0.8) (layer F.Cu) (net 26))
 (segment (start 146.304 47.244) (end 133.858 47.244) (width 0.8) (layer F.Cu) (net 26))
 (segment (start 159.512 45.72) (end 147.32 45.72) (width 0.8) (layer F.Cu) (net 27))
 (segment (start 147.32 45.72) (end 146.304 44.704) (width 0.8) (layer F.Cu) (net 27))
 (segment (start 146.304 44.704) (end 133.858 44.704) (width 0.8) (layer F.Cu) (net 27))
 (segment (start 159.512 43.18) (end 147.32 43.18) (width 0.8) (layer F.Cu) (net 28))
 (segment (start 147.32 43.18) (end 146.304 42.164) (width 0.8) (layer F.Cu) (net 28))
 (segment (start 146.304 42.164) (end 133.858 42.164) (width 0.8) (layer F.Cu) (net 28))
 (segment (start 159.512 40.64) (end 147.32 40.64) (width 0.8) (layer F.Cu) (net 29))
 (segment (start 147.32 40.64) (end 146.304 39.624) (width 0.8) (layer F.Cu) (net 29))
 (segment (start 146.304 39.624) (end 133.858 39.624) (width 0.8) (layer F.Cu) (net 29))
 (segment (start 159.512 38.1) (end 147.32 38.1) (width 0.8) (layer F.Cu) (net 30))
 (segment (start 147.32 38.1) (end 146.304 37.084) (width 0.8) (layer F.Cu) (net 30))
 (segment (start 146.304 37.084) (end 133.858 37.084) (width 0.8) (layer F.Cu) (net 30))
 (segment (start 159.512 35.56) (end 147.32 35.56) (width 0.8) (layer F.Cu) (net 31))
 (segment (start 147.32 35.56) (end 146.304 34.544) (width 0.8) (layer F.Cu) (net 31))
 (segment (start 146.304 34.544) (end 133.858 34.544) (width 0.8) (layer F.Cu) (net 31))
 (segment (start 159.512 57.658) (end 159.512 58.42) (width 0.4) (layer F.Cu) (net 33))
 (segment (start 154.178 52.324) (end 159.512 57.658) (width 0.4) (layer F.Cu) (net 33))
 (segment (start 133.858 52.324) (end 154.178 52.324) (width 0.4) (layer F.Cu) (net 33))
 (segment (start 159.512 68.58) (end 159.512 58.42) (width 0.4) (layer F.Cu) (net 33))
 (segment (start 157.410001 71.558001) (end 156.972 71.12) (width 0.4) (layer F.Cu) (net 34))
 (segment (start 156.972 71.12) (end 156.972 73.168) (width 0.8) (layer F.Cu) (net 34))
 (segment (start 135.382 75.438) (end 135.382 77.978) (width 0.8) (layer F.Cu) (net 2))
 (segment (start 135.382 77.978) (end 135.382 76.328) (width 0.8) (layer F.Cu) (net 2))
 (segment (start 135.382 75.438) (end 135.382 71.12) (width 0.8) (layer F.Cu) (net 2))
 (segment (start 139.192 71.12) (end 135.382 71.12) (width 0.8) (layer F.Cu) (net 2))
 (segment (start 134.62 61.722) (end 134.62 64.77) (width 0.8) (layer F.Cu) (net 2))
 (segment (start 133.858 32.004) (end 135.128 32.004) (width 0.8) (layer F.Cu) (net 2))
 (segment (start 135.128 32.004) (end 136.144 30.988) (width 0.8) (layer F.Cu) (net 2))
 (segment (start 136.144 30.988) (end 136.144 24.384) (width 0.8) (layer F.Cu) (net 2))
 (segment (start 134.62 22.86) (end 129.032 22.86) (width 0.8) (layer F.Cu) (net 2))
 (segment (start 136.144 24.384) (end 134.62 22.86) (width 0.8) (layer F.Cu) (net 2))
 (segment (start 132.56598 54.07998) (end 131.318 52.832) (width 0.8) (layer F.Cu) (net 2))
 (segment (start 150.09198 54.07998) (end 132.56598 54.07998) (width 0.8) (layer F.Cu) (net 2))
 (segment (start 152.560636 56.548636) (end 150.09198 54.07998) (width 0.8) (layer F.Cu) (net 2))
 (segment (start 131.318 52.832) (end 131.318 33.274) (width 0.8) (layer F.Cu) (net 2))
 (segment (start 152.560636 63.991591) (end 152.560636 56.548636) (width 0.8) (layer F.Cu) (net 2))
 (segment (start 151.180198 65.372029) (end 152.560636 63.991591) (width 0.8) (layer F.Cu) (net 2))
 (segment (start 131.318 33.274) (end 132.588 32.004) (width 0.8) (layer F.Cu) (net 2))
 (segment (start 138.589971 65.372029) (end 151.180198 65.372029) (width 0.8) (layer F.Cu) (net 2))
 (segment (start 137.995999 65.966001) (end 138.589971 65.372029) (width 0.8) (layer F.Cu) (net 2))
 (segment (start 136.463999 65.966001) (end 137.995999 65.966001) (width 0.8) (layer F.Cu) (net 2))
 (segment (start 135.013998 64.516) (end 136.463999 65.966001) (width 0.8) (layer F.Cu) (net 2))
 (segment (start 132.588 32.004) (end 133.858 32.004) (width 0.8) (layer F.Cu) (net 2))
 (segment (start 134.62 64.516) (end 135.013998 64.516) (width 0.8) (layer F.Cu) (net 2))
 (segment (start 134.189469 66.807467) (end 134.868533 66.807467) (width 0.4) (layer F.Cu) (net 12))
 (segment (start 129.592003 62.210001) (end 134.189469 66.807467) (width 0.4) (layer F.Cu) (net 12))
 (segment (start 127.742001 62.210001) (end 129.592003 62.210001) (width 0.4) (layer F.Cu) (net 12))
 (segment (start 138.285917 66.807467) (end 134.868533 66.807467) (width 0.4) (layer F.Cu) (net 12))
 (segment (start 156.972 53.34) (end 159.512 53.34) (width 0.8) (layer F.Cu) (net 24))
 (segment (start 153.416 49.784) (end 156.972 53.34) (width 0.8) (layer F.Cu) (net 24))
 (segment (start 133.858 49.784) (end 153.416 49.784) (width 0.8) (layer F.Cu) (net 24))
 (segment (start 148.911949 82.228051) (end 153.162 77.978) (width 0.4) (layer F.Cu) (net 5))
 (segment (start 132.687509 82.228051) (end 148.911949 82.228051) (width 0.4) (layer F.Cu) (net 5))
 (segment (start 130.349955 79.890497) (end 132.687509 82.228051) (width 0.4) (layer F.Cu) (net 5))
 (segment (start 130.349955 70.405955) (end 130.349955 79.890497) (width 0.4) (layer F.Cu) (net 5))
 (segment (start 129.774001 69.830001) (end 130.349955 70.405955) (width 0.4) (layer F.Cu) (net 5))
 (segment (start 127.742001 69.830001) (end 129.774001 69.830001) (width 0.4) (layer F.Cu) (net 5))
 (segment (start 126.492 68.58) (end 127.742001 69.830001) (width 0.4) (layer F.Cu) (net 5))
 (segment (start 129.032 68.58) (end 130.441963 68.58) (width 0.4) (layer F.Cu) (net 7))
 (segment (start 130.441963 68.58) (end 130.949964 69.088001) (width 0.4) (layer F.Cu) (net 7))
 (segment (start 130.949964 69.088001) (end 130.949964 79.641964) (width 0.4) (layer F.Cu) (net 7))
 (segment (start 146.971959 81.628041) (end 150.622 77.978) (width 0.4) (layer F.Cu) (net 7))
 (segment (start 132.936041 81.628041) (end 146.971959 81.628041) (width 0.4) (layer F.Cu) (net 7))
 (segment (start 130.949964 79.641964) (end 132.936041 81.628041) (width 0.4) (layer F.Cu) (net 7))
 (segment (start 127.781999 67.329999) (end 131.078375 67.329999) (width 0.4) (layer F.Cu) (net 9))
 (segment (start 126.492 66.04) (end 127.781999 67.329999) (width 0.4) (layer F.Cu) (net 9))
 (segment (start 131.549972 67.801596) (end 131.549973 79.231599) (width 0.4) (layer F.Cu) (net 9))
 (segment (start 131.078375 67.329999) (end 131.549972 67.801596) (width 0.4) (layer F.Cu) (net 9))
 (segment (start 145.031969 81.028031) (end 148.082 77.978) (width 0.4) (layer F.Cu) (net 9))
 (segment (start 133.346405 81.028031) (end 145.031969 81.028031) (width 0.4) (layer F.Cu) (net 9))
 (segment (start 131.549973 79.231599) (end 133.346405 81.028031) (width 0.4) (layer F.Cu) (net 9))
 (segment (start 144.107979 80.428021) (end 145.542 78.994) (width 0.4) (layer F.Cu) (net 11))
 (segment (start 133.594937 80.428021) (end 144.107979 80.428021) (width 0.4) (layer F.Cu) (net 11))
 (segment (start 145.542 78.994) (end 145.542 77.978) (width 0.4) (layer F.Cu) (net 11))
 (segment (start 132.149982 78.983066) (end 133.594937 80.428021) (width 0.4) (layer F.Cu) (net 11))
 (segment (start 132.149982 67.553064) (end 132.149982 78.983066) (width 0.4) (layer F.Cu) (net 11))
 (segment (start 130.636918 66.04) (end 132.149982 67.553064) (width 0.4) (layer F.Cu) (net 11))
 (segment (start 129.032 66.04) (end 130.636918 66.04) (width 0.4) (layer F.Cu) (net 11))
 (segment (start 141.151989 79.828011) (end 143.002 77.978) (width 0.4) (layer F.Cu) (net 13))
 (segment (start 133.843469 79.828011) (end 141.151989 79.828011) (width 0.4) (layer F.Cu) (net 13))
 (segment (start 132.749991 78.734533) (end 133.843469 79.828011) (width 0.4) (layer F.Cu) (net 13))
 (segment (start 132.74999 67.304532) (end 132.749991 78.734533) (width 0.4) (layer F.Cu) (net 13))
 (segment (start 130.235457 64.789999) (end 132.74999 67.304532) (width 0.4) (layer F.Cu) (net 13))
 (segment (start 127.781999 64.789999) (end 130.235457 64.789999) (width 0.4) (layer F.Cu) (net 13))
 (segment (start 126.492 63.5) (end 127.781999 64.789999) (width 0.4) (layer F.Cu) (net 13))
 (segment (start 133.35 78.486) (end 134.092001 79.228001) (width 0.4) (layer F.Cu) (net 15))
 (segment (start 133.35 67.056) (end 133.35 78.486) (width 0.4) (layer F.Cu) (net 15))
 (segment (start 134.092001 79.228001) (end 139.211999 79.228001) (width 0.4) (layer F.Cu) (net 15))
 (segment (start 129.794 63.5) (end 133.35 67.056) (width 0.4) (layer F.Cu) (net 15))
 (segment (start 139.211999 79.228001) (end 140.462 77.978) (width 0.4) (layer F.Cu) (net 15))
 (segment (start 129.032 63.5) (end 129.794 63.5) (width 0.4) (layer F.Cu) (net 15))
 (segment (start 157.34137 77.216) (end 156.21 77.216) (width 0.4) (layer F.Cu) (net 3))
 (segment (start 160.762001 73.795369) (end 157.34137 77.216) (width 0.4) (layer F.Cu) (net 3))
 (segment (start 160.762001 69.869999) (end 160.762001 73.795369) (width 0.4) (layer F.Cu) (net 3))
 (segment (start 162.052 68.58) (end 160.762001 69.869999) (width 0.4) (layer F.Cu) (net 3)))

